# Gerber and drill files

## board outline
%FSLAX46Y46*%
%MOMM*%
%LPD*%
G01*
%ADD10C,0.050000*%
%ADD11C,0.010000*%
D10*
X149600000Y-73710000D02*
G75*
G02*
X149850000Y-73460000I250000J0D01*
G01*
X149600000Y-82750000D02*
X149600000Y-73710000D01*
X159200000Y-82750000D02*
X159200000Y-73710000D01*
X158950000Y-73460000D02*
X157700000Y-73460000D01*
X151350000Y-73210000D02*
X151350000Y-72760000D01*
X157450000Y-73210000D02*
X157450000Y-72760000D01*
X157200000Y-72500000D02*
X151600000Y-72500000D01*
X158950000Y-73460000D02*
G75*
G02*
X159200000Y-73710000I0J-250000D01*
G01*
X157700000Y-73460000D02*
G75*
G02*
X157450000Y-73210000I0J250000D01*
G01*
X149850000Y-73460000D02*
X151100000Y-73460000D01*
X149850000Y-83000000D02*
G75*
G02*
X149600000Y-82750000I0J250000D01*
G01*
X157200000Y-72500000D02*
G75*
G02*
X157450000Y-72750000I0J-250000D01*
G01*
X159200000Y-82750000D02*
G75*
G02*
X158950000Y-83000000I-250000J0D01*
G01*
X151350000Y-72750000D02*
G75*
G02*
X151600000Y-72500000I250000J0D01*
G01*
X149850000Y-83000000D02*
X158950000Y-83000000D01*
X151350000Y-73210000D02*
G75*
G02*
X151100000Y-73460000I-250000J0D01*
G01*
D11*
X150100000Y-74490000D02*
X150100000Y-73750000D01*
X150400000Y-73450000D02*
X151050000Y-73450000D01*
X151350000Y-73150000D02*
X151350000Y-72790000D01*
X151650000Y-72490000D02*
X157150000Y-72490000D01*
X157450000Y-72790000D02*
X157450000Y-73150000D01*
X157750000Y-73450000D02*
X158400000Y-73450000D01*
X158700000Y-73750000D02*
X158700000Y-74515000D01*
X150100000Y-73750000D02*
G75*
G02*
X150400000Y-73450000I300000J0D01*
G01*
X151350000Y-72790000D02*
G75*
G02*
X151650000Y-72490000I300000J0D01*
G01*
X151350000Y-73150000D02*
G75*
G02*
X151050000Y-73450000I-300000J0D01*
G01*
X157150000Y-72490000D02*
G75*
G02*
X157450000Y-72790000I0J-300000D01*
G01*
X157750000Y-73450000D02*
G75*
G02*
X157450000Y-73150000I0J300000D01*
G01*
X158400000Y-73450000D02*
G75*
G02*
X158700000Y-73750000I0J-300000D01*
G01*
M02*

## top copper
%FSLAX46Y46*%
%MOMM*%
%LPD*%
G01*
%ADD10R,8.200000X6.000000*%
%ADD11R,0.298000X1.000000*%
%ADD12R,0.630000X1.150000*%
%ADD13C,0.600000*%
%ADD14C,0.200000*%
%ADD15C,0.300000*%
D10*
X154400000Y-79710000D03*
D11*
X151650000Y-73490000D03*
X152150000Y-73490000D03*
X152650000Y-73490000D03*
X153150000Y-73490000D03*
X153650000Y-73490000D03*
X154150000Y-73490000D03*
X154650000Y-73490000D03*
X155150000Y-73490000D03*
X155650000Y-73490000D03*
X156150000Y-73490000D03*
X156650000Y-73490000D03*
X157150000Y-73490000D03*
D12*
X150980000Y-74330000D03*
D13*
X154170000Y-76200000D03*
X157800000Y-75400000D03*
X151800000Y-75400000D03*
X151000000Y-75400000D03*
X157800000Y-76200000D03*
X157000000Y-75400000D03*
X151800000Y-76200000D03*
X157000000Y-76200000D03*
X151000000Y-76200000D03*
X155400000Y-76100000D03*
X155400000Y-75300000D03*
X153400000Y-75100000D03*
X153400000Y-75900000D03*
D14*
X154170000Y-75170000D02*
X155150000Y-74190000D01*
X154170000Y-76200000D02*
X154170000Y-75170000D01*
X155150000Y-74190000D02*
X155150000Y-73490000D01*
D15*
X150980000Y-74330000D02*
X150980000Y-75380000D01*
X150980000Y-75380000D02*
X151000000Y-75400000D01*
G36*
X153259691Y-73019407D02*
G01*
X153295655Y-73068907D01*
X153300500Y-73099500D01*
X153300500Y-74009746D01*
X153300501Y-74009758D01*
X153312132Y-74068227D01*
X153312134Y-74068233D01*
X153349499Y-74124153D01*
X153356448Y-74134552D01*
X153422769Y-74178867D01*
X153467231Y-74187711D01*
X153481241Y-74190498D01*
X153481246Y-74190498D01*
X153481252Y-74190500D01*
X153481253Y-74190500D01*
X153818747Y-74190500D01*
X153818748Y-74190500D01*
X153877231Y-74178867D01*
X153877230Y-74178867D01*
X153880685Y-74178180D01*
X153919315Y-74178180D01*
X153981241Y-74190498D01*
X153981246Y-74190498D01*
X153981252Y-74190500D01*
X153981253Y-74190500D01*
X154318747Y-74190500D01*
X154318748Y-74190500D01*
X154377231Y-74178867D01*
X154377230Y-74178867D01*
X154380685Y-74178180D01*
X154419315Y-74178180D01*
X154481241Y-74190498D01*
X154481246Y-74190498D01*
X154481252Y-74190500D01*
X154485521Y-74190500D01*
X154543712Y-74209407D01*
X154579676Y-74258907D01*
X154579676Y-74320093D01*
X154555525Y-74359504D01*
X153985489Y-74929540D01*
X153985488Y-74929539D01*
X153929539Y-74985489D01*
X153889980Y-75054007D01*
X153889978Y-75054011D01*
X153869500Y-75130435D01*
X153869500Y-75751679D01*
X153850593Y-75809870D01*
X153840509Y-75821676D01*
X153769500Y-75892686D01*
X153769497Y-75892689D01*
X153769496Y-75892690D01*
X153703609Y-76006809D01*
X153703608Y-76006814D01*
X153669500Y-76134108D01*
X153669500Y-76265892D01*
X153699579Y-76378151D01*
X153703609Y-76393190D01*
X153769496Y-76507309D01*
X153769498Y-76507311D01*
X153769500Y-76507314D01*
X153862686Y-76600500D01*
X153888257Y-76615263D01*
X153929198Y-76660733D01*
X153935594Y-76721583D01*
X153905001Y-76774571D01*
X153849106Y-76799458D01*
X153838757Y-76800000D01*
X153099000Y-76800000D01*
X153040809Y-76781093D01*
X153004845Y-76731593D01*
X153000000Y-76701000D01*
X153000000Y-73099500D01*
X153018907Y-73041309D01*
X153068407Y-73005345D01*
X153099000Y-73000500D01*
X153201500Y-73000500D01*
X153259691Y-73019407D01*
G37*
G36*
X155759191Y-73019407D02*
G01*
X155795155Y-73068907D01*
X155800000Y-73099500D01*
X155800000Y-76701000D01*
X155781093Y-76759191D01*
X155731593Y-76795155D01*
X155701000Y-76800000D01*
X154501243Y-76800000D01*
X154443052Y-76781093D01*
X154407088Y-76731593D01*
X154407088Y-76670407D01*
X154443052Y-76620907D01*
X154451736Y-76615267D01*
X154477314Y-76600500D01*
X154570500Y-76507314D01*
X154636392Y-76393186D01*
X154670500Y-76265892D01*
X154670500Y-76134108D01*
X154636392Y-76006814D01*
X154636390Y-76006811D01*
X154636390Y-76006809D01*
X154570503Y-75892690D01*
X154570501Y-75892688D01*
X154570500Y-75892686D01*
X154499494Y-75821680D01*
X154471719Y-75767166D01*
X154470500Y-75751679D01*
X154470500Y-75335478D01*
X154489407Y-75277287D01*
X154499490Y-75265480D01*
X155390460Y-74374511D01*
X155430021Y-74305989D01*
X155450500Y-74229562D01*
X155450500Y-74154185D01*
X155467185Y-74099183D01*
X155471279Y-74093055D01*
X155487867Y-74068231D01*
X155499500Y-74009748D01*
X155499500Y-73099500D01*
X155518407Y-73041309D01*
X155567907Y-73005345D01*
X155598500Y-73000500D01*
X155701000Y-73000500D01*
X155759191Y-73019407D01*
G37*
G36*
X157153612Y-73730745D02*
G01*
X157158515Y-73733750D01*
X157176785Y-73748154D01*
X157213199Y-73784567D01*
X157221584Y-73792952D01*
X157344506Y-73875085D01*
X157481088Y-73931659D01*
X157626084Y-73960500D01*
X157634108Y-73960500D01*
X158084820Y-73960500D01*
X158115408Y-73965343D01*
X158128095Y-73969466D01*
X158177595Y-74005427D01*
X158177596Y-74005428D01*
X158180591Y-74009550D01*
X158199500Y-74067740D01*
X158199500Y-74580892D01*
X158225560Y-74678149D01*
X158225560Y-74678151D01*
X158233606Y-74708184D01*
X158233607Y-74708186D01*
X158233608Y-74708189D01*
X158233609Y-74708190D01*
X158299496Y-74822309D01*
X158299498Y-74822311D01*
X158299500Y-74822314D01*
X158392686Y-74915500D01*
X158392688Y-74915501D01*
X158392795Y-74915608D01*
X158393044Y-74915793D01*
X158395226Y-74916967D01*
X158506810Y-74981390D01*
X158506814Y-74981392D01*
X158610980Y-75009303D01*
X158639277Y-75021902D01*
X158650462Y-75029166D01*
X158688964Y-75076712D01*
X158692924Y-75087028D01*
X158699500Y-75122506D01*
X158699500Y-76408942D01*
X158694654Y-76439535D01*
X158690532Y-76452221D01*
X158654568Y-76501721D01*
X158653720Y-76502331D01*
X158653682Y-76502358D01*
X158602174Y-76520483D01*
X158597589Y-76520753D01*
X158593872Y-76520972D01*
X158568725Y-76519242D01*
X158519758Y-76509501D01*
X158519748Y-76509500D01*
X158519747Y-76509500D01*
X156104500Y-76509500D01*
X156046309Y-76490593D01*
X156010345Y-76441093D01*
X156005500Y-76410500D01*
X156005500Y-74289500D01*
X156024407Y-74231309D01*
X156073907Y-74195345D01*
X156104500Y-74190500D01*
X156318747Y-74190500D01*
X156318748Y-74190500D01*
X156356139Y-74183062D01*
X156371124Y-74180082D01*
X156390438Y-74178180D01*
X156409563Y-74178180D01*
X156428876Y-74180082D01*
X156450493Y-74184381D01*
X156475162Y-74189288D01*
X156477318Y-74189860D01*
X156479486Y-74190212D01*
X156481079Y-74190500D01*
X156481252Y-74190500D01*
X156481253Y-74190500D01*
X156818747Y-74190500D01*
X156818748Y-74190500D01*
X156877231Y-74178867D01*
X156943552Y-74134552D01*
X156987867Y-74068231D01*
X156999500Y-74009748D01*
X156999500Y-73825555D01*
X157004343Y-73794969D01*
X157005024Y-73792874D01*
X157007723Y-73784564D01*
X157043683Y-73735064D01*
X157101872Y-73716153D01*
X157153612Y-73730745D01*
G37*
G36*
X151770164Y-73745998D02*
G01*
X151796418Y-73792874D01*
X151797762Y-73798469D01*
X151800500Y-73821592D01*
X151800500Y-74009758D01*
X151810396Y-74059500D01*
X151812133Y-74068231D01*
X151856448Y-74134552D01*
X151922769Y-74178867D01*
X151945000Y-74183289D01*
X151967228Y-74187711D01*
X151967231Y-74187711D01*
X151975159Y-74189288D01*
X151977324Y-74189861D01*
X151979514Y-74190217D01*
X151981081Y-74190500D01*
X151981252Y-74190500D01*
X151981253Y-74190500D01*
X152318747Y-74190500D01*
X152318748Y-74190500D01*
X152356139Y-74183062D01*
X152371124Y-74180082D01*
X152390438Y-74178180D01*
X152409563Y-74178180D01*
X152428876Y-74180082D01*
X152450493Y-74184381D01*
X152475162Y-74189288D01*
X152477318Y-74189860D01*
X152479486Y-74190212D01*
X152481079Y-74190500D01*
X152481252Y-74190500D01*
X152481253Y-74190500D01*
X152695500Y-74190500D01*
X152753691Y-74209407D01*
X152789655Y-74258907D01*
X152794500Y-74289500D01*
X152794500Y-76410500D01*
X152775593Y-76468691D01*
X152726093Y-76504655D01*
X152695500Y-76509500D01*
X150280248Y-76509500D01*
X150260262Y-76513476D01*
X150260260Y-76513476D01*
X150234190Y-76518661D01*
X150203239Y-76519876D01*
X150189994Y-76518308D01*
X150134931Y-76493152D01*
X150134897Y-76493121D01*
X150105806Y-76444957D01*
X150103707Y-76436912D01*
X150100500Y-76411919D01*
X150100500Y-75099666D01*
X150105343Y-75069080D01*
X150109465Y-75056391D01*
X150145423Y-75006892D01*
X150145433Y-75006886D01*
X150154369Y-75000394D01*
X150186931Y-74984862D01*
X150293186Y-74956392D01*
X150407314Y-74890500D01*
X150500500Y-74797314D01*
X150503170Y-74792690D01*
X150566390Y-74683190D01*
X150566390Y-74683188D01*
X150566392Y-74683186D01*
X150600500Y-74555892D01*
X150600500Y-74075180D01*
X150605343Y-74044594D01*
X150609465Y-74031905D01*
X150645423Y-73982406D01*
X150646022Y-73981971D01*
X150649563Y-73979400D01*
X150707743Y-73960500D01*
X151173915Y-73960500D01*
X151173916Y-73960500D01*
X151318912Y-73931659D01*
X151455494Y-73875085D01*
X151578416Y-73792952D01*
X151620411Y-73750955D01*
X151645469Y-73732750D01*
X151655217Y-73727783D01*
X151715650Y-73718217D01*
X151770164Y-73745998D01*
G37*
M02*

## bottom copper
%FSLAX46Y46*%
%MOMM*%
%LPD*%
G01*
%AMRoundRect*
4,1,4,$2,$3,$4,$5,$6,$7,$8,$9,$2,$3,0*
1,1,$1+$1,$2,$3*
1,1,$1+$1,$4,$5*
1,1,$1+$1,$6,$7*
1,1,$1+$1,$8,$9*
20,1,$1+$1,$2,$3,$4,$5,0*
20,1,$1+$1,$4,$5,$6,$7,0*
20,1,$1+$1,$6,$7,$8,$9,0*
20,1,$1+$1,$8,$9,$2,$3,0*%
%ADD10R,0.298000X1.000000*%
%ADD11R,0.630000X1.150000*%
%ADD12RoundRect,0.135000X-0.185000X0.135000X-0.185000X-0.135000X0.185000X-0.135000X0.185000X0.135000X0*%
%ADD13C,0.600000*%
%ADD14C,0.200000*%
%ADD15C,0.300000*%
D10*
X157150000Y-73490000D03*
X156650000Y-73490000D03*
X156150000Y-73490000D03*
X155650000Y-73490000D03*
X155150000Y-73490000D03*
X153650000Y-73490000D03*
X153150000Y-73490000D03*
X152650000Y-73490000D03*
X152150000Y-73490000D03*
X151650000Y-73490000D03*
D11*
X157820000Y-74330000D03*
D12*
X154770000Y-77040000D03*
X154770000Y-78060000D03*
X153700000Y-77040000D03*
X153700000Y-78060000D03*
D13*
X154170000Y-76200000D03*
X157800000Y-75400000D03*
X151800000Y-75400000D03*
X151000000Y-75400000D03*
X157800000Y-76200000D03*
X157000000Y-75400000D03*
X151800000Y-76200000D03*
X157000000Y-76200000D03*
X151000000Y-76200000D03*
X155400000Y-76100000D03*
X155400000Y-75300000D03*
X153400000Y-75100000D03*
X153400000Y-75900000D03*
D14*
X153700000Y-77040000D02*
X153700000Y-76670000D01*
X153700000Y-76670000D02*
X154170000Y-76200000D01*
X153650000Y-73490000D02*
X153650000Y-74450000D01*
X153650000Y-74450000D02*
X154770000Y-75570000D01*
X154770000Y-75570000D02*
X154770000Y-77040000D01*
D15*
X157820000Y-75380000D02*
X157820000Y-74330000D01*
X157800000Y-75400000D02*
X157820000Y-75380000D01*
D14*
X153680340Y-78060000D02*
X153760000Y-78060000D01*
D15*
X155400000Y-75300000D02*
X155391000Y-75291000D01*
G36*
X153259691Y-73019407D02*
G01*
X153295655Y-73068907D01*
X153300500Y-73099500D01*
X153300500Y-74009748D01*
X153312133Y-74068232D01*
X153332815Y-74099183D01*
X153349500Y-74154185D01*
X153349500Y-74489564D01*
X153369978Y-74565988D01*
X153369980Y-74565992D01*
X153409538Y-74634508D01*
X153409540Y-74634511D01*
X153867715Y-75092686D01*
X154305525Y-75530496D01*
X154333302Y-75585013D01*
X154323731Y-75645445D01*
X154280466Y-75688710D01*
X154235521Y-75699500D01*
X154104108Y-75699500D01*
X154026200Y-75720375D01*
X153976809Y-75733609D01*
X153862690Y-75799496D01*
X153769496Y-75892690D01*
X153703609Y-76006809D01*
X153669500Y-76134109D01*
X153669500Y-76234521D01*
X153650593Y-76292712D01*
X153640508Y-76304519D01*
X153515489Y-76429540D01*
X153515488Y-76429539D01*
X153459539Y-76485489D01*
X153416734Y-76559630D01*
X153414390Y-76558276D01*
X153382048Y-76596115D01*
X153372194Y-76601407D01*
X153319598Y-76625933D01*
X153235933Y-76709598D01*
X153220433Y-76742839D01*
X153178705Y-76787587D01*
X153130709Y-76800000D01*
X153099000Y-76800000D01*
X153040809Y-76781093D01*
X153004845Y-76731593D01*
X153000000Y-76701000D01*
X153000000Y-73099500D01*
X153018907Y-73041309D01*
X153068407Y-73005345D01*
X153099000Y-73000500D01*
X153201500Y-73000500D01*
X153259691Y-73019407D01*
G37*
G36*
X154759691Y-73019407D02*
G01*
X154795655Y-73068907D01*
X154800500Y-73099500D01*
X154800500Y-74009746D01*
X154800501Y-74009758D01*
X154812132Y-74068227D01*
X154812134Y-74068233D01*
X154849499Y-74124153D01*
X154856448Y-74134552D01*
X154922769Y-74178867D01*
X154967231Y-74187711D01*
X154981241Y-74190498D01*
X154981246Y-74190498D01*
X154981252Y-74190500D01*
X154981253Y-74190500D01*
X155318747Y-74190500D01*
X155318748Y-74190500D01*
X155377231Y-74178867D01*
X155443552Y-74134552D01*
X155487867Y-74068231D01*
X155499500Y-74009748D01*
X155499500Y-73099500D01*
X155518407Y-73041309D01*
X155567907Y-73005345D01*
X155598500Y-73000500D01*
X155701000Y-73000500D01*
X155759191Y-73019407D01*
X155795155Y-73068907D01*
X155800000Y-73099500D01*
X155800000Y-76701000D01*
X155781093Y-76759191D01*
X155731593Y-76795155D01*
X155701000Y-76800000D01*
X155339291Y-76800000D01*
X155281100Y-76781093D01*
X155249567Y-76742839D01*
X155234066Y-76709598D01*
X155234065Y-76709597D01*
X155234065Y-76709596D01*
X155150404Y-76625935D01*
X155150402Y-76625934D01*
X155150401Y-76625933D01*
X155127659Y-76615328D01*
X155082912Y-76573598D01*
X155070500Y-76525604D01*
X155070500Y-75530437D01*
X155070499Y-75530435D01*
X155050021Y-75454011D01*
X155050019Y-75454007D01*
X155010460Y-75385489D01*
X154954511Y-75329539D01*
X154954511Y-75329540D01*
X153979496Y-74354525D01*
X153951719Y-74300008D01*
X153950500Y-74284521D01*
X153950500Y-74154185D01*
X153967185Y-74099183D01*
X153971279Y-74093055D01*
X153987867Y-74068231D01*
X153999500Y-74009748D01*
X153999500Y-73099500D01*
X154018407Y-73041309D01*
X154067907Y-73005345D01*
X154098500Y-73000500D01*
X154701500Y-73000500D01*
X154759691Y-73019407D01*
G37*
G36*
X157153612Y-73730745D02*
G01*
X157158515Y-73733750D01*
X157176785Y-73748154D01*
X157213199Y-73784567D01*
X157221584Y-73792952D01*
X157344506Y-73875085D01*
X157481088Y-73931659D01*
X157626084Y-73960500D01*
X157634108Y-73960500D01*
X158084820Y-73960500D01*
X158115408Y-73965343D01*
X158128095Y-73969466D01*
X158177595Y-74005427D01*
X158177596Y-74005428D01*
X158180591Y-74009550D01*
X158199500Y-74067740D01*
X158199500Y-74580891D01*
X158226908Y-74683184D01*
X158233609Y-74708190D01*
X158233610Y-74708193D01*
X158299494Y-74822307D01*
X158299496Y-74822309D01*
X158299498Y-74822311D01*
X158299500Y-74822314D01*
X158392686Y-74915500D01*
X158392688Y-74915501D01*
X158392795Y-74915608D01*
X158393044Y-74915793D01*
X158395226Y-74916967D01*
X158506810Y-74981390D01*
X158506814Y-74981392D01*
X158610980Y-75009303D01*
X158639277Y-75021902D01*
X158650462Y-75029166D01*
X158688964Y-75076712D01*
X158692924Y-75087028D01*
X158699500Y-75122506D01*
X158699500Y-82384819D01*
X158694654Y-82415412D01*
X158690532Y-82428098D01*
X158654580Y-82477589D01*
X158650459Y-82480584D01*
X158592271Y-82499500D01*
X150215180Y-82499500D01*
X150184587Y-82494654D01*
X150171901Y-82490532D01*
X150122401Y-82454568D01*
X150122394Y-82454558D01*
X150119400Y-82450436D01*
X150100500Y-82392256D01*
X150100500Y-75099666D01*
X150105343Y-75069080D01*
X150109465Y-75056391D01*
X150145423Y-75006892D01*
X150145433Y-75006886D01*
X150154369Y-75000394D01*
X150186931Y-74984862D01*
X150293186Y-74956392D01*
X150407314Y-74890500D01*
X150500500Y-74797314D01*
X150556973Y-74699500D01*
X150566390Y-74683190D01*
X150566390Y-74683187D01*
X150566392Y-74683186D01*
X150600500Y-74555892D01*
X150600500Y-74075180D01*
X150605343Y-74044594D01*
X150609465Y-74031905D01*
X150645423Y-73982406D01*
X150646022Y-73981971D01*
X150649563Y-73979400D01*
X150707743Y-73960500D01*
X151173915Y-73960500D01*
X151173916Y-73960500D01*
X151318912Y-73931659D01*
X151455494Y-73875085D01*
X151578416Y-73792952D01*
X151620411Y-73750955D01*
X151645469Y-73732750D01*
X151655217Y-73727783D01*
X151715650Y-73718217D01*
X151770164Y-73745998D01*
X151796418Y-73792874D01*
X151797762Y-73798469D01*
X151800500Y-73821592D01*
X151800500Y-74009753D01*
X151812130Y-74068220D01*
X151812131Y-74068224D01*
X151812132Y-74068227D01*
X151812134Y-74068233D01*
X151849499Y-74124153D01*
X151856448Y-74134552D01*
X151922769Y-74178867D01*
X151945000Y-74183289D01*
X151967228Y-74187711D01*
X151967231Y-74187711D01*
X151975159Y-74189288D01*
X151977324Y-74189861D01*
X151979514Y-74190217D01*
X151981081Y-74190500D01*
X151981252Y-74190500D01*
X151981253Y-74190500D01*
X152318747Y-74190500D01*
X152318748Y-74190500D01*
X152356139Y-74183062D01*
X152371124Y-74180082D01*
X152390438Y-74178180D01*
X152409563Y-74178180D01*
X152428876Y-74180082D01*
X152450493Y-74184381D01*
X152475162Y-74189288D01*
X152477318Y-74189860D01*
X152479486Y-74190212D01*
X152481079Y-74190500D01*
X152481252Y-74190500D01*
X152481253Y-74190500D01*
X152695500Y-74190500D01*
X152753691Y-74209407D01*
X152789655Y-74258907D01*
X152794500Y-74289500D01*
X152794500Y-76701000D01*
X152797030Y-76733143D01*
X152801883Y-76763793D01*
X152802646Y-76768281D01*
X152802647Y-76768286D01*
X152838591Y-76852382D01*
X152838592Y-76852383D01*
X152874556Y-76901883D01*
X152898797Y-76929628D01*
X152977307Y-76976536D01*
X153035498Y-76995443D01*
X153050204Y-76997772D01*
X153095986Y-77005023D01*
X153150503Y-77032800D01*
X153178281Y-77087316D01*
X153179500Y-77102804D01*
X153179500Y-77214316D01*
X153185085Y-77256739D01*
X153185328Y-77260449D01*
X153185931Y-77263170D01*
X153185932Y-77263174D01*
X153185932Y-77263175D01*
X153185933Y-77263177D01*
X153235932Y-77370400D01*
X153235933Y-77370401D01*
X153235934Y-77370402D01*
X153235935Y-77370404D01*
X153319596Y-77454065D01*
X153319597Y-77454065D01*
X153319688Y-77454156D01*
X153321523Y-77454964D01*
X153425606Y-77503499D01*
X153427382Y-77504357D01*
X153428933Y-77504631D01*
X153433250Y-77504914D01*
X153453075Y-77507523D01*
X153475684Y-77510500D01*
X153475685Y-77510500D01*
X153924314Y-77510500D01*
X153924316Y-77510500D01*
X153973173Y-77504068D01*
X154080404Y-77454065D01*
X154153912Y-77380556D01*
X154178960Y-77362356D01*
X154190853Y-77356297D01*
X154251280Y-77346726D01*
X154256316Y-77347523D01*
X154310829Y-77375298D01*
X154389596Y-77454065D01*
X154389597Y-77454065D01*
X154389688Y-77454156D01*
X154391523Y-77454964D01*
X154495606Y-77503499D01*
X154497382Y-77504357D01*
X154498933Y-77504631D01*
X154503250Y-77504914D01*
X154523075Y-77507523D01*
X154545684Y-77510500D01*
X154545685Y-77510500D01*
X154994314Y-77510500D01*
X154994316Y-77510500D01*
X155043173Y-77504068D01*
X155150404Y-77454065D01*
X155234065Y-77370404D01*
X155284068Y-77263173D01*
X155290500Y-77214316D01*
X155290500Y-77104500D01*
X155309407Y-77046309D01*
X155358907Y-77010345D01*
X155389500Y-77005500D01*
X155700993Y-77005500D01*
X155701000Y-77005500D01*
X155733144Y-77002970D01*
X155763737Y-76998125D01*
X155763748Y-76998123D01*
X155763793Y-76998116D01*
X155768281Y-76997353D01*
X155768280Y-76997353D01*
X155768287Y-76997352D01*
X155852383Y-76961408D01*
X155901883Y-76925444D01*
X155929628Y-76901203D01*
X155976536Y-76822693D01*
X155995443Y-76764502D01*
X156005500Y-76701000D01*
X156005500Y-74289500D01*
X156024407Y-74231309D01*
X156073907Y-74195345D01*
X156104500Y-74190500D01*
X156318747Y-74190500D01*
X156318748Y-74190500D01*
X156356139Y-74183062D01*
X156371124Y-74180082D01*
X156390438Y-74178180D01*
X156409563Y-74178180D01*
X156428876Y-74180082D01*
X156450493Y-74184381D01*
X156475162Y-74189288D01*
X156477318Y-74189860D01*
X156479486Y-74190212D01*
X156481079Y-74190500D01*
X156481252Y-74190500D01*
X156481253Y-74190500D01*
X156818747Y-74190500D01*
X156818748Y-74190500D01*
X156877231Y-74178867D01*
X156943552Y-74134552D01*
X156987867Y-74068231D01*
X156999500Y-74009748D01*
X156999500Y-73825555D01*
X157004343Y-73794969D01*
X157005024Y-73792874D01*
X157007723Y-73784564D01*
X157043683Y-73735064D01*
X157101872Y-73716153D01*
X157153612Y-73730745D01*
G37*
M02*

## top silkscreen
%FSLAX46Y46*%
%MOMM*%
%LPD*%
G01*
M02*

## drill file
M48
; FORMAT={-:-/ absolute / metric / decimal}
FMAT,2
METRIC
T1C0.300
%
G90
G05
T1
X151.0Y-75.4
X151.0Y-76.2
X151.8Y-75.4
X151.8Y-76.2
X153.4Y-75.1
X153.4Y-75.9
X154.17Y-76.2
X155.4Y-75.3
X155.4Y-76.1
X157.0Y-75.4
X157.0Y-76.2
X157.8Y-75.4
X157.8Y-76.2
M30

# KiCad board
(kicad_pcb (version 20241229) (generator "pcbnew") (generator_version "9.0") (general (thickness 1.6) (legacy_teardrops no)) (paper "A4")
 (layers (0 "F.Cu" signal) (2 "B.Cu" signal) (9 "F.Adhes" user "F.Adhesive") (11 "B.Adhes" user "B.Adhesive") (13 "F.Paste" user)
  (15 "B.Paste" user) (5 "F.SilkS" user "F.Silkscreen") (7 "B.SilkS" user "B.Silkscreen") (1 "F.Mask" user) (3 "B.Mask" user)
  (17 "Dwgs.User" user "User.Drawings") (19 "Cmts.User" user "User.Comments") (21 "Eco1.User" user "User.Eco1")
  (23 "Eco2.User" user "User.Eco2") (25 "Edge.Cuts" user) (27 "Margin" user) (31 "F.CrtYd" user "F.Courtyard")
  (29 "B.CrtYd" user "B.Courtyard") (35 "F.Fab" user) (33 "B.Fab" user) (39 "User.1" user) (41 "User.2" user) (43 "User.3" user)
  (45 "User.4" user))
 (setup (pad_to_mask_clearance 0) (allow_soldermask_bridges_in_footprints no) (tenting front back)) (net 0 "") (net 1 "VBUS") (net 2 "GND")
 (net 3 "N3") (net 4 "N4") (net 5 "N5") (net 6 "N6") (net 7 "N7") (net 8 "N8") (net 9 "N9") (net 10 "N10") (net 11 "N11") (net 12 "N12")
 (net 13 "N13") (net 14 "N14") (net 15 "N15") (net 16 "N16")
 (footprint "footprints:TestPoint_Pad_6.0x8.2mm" (layer "F.Cu") (at 154.3 79.81)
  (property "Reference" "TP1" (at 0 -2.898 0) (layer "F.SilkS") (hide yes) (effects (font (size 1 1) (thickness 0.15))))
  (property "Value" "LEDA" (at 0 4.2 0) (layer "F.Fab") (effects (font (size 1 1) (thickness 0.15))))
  (pad "1" smd rect (at 0.1 -0.1) (size 8.2 6) (layers "F.Cu" "F.Mask") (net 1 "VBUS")))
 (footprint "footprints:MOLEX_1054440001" (layer "F.Cu") (at 154.4 72.49 180)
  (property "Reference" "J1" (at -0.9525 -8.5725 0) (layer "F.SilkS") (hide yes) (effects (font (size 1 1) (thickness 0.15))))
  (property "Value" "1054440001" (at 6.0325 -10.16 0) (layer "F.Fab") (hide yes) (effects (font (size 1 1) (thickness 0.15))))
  (fp_line (start 4.3 -2) (end 4.3 -1.26) (stroke (width 0.01) (type solid)) (layer "Edge.Cuts"))
  (fp_line (start 4 -0.96) (end 3.35 -0.96) (stroke (width 0.01) (type solid)) (layer "Edge.Cuts"))
  (fp_line (start 3.05 -0.66) (end 3.05 -0.3) (stroke (width 0.01) (type solid)) (layer "Edge.Cuts"))
  (fp_line (start 2.75 0) (end -2.75 0) (stroke (width 0.01) (type solid)) (layer "Edge.Cuts"))
  (fp_line (start -3.05 -0.3) (end -3.05 -0.66) (stroke (width 0.01) (type solid)) (layer "Edge.Cuts"))
  (fp_line (start -3.35 -0.96) (end -4 -0.96) (stroke (width 0.01) (type solid)) (layer "Edge.Cuts"))
  (fp_line (start -4.3 -1.26) (end -4.3 -2.025) (stroke (width 0.01) (type solid)) (layer "Edge.Cuts"))
  (fp_arc (start 4.3 -1.26) (mid 4.212132 -1.047868) (end 4 -0.96) (stroke (width 0.01) (type solid)) (layer "Edge.Cuts"))
  (fp_arc (start 3.05 -0.3) (mid 2.962132 -0.087868) (end 2.75 0) (stroke (width 0.01) (type solid)) (layer "Edge.Cuts"))
  (fp_arc (start 3.05 -0.66) (mid 3.137868 -0.872132) (end 3.35 -0.96) (stroke (width 0.01) (type solid)) (layer "Edge.Cuts"))
  (fp_arc (start -2.75 0) (mid -2.962132 -0.087868) (end -3.05 -0.3) (stroke (width 0.01) (type solid)) (layer "Edge.Cuts"))
  (fp_arc (start -3.35 -0.96) (mid -3.137868 -0.872132) (end -3.05 -0.66) (stroke (width 0.01) (type solid)) (layer "Edge.Cuts"))
  (fp_arc (start -4 -0.96) (mid -4.212132 -1.047868) (end -4.3 -1.26) (stroke (width 0.01) (type solid)) (layer "Edge.Cuts"))
  (pad "A1" smd rect (at 2.75 -1 180) (size 0.298 1) (layers "F.Cu" "F.Paste") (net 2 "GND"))
  (pad "A2" smd rect (at 2.25 -1 180) (size 0.298 1) (layers "F.Cu" "F.Paste") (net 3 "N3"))
  (pad "A3" smd rect (at 1.75 -1 180) (size 0.298 1) (layers "F.Cu" "F.Paste") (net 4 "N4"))
  (pad "A4" smd rect (at 1.25 -1 180) (size 0.298 1) (layers "F.Cu" "F.Paste") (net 1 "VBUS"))
  (pad "A5" smd rect (at 0.75 -1 180) (size 0.298 1) (layers "F.Cu" "F.Paste") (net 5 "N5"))
  (pad "A6" smd rect (at 0.25 -1 180) (size 0.298 1) (layers "F.Cu" "F.Paste") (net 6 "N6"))
  (pad "A7" smd rect (at -0.25 -1 180) (size 0.298 1) (layers "F.Cu" "F.Paste") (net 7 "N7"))
  (pad "A8" smd rect (at -0.75 -1 180) (size 0.298 1) (layers "F.Cu" "F.Paste") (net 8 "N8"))
  (pad "A9" smd rect (at -1.25 -1 180) (size 0.298 1) (layers "F.Cu" "F.Paste") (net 1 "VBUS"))
  (pad "A10" smd rect (at -1.75 -1 180) (size 0.298 1) (layers "F.Cu" "F.Paste") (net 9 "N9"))
  (pad "A11" smd rect (at -2.25 -1 180) (size 0.298 1) (layers "F.Cu" "F.Paste") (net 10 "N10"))
  (pad "A12" smd rect (at -2.75 -1 180) (size 0.298 1) (layers "F.Cu" "F.Paste") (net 2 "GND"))
  (pad "B1" smd rect (at -2.75 -1 180) (size 0.298 1) (layers "B.Cu" "B.Paste") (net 2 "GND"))
  (pad "B2" smd rect (at -2.25 -1 180) (size 0.298 1) (layers "B.Cu" "B.Paste") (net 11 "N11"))
  (pad "B3" smd rect (at -1.75 -1 180) (size 0.298 1) (layers "B.Cu" "B.Paste") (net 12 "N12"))
  (pad "B4" smd rect (at -1.25 -1 180) (size 0.298 1) (layers "B.Cu" "B.Paste") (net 1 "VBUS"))
  (pad "B5" smd rect (at -0.75 -1 180) (size 0.298 1) (layers "B.Cu" "B.Paste") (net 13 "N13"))
  (pad "B8" smd rect (at 0.75 -1 180) (size 0.298 1) (layers "B.Cu" "B.Paste") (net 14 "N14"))
  (pad "B9" smd rect (at 1.25 -1 180) (size 0.298 1) (layers "B.Cu" "B.Paste") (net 1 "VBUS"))
  (pad "B10" smd rect (at 1.75 -1 180) (size 0.298 1) (layers "B.Cu" "B.Paste") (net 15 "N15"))
  (pad "B11" smd rect (at 2.25 -1 180) (size 0.298 1) (layers "B.Cu" "B.Paste") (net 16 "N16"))
  (pad "B12" smd rect (at 2.75 -1 180) (size 0.298 1) (layers "B.Cu" "B.Paste") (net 2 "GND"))
  (pad "SH1" smd rect (at 3.42 -1.84 180) (size 0.63 1.15) (layers "F.Cu" "F.Paste") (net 2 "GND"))
  (pad "SH2" smd rect (at -3.42 -1.84 180) (size 0.63 1.15) (layers "B.Cu" "B.Paste") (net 2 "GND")))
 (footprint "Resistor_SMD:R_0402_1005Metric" (layer "B.Cu") (at 154.77 77.55 -90)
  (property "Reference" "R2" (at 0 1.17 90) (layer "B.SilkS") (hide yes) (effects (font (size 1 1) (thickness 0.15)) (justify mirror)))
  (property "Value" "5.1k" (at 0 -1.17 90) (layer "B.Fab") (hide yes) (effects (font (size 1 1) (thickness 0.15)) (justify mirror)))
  (pad "1" smd roundrect (at -0.51 0 270) (size 0.54 0.64) (layers "B.Cu" "B.Mask" "B.Paste") (roundrect_rratio 0.25) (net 14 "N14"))
  (pad "2" smd roundrect (at 0.51 0 270) (size 0.54 0.64) (layers "B.Cu" "B.Mask" "B.Paste") (roundrect_rratio 0.25) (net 2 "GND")))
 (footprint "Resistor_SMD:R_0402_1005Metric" (layer "B.Cu") (at 153.7 77.55 -90)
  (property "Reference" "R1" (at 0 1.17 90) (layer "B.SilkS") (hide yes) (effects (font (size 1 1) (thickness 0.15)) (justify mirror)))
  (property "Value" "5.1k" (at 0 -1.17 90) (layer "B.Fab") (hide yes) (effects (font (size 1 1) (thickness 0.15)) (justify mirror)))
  (pad "1" smd roundrect (at -0.51 0 270) (size 0.54 0.64) (layers "B.Cu" "B.Mask" "B.Paste") (roundrect_rratio 0.25) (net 8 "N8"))
  (pad "2" smd roundrect (at 0.51 0 270) (size 0.54 0.64) (layers "B.Cu" "B.Mask" "B.Paste") (roundrect_rratio 0.25) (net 2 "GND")))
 (gr_arc (start 149.6 73.71) (mid 149.673223 73.533223) (end 149.85 73.46) (stroke (width 0.05) (type default)) (layer "Edge.Cuts"))
 (gr_line (start 149.6 82.75) (end 149.6 73.71) (stroke (width 0.05) (type solid)) (layer "Edge.Cuts"))
 (gr_line (start 159.2 82.75) (end 159.2 73.71) (stroke (width 0.05) (type solid)) (layer "Edge.Cuts"))
 (gr_line (start 158.95 73.46) (end 157.7 73.46) (stroke (width 0.05) (type solid)) (layer "Edge.Cuts"))
 (gr_line (start 151.35 73.21) (end 151.35 72.76) (stroke (width 0.05) (type solid)) (layer "Edge.Cuts"))
 (gr_line (start 157.45 73.21) (end 157.45 72.76) (stroke (width 0.05) (type solid)) (layer "Edge.Cuts"))
 (gr_line (start 157.2 72.5) (end 151.6 72.5) (stroke (width 0.05) (type default)) (layer "Edge.Cuts"))
 (gr_arc (start 158.95 73.46) (mid 159.126777 73.533223) (end 159.2 73.71) (stroke (width 0.05) (type default)) (layer "Edge.Cuts"))
 (gr_arc (start 157.7 73.46) (mid 157.523223 73.386777) (end 157.45 73.21) (stroke (width 0.05) (type default)) (layer "Edge.Cuts"))
 (gr_line (start 149.85 73.46) (end 151.1 73.46) (stroke (width 0.05) (type solid)) (layer "Edge.Cuts"))
 (gr_arc (start 149.85 83) (mid 149.673223 82.926777) (end 149.6 82.75) (stroke (width 0.05) (type default)) (layer "Edge.Cuts"))
 (gr_arc (start 157.2 72.5) (mid 157.376777 72.573223) (end 157.45 72.75) (stroke (width 0.05) (type default)) (layer "Edge.Cuts"))
 (gr_arc (start 159.2 82.75) (mid 159.126777 82.926777) (end 158.95 83) (stroke (width 0.05) (type default)) (layer "Edge.Cuts"))
 (gr_arc (start 151.35 72.75) (mid 151.423223 72.573223) (end 151.6 72.5) (stroke (width 0.05) (type default)) (layer "Edge.Cuts"))
 (gr_line (start 149.85 83) (end 158.95 83) (stroke (width 0.05) (type default)) (layer "Edge.Cuts"))
 (gr_arc (start 151.35 73.21) (mid 151.276777 73.386777) (end 151.1 73.46) (stroke (width 0.05) (type default)) (layer "Edge.Cuts"))
 (segment (start 154.17 75.17) (end 155.15 74.19) (width 0.2) (layer "F.Cu") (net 8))
 (segment (start 154.17 76.2) (end 154.17 75.17) (width 0.2) (layer "F.Cu") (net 8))
 (segment (start 155.15 74.19) (end 155.15 73.49) (width 0.2) (layer "F.Cu") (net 8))
 (via (at 154.17 76.2) (size 0.6) (drill 0.3) (layers "F.Cu" "B.Cu") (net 8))
 (segment (start 153.7 77.04) (end 153.7 76.67) (width 0.2) (layer "B.Cu") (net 8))
 (segment (start 153.7 76.67) (end 154.17 76.2) (width 0.2) (layer "B.Cu") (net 8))
 (segment (start 153.65 73.49) (end 153.65 74.45) (width 0.2) (layer "B.Cu") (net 14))
 (segment (start 153.65 74.45) (end 154.77 75.57) (width 0.2) (layer "B.Cu") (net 14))
 (segment (start 154.77 75.57) (end 154.77 77.04) (width 0.2) (layer "B.Cu") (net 14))
 (segment (start 150.98 74.33) (end 150.98 75.38) (width 0.3) (layer "F.Cu") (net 2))
 (segment (start 150.98 75.38) (end 151 75.4) (width 0.3) (layer "F.Cu") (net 2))
 (via (at 157.8 75.4) (size 0.6) (drill 0.3) (layers "F.Cu" "B.Cu") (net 2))
 (via (at 151.8 75.4) (size 0.6) (drill 0.3) (layers "F.Cu" "B.Cu") (free yes) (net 2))
 (via (at 151 75.4) (size 0.6) (drill 0.3) (layers "F.Cu" "B.Cu") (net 2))
 (via (at 157.8 76.2) (size 0.6) (drill 0.3) (layers "F.Cu" "B.Cu") (free yes) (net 2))
 (via (at 157 75.4) (size 0.6) (drill 0.3) (layers "F.Cu" "B.Cu") (free yes) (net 2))
 (via (at 151.8 76.2) (size 0.6) (drill 0.3) (layers "F.Cu" "B.Cu") (free yes) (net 2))
 (via (at 157 76.2) (size 0.6) (drill 0.3) (layers "F.Cu" "B.Cu") (free yes) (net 2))
 (via (at 151 76.2) (size 0.6) (drill 0.3) (layers "F.Cu" "B.Cu") (free yes) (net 2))
 (segment (start 157.82 75.38) (end 157.82 74.33) (width 0.3) (layer "B.Cu") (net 2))
 (segment (start 157.8 75.4) (end 157.82 75.38) (width 0.3) (layer "B.Cu") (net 2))
 (segment (start 153.68034 78.06) (end 153.76 78.06) (width 0.2) (layer "B.Cu") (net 2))
 (via (at 155.4 76.1) (size 0.6) (drill 0.3) (layers "F.Cu" "B.Cu") (free yes) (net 1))
 (via (at 155.4 75.3) (size 0.6) (drill 0.3) (layers "F.Cu" "B.Cu") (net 1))
 (via (at 153.4 75.1) (size 0.6) (drill 0.3) (layers "F.Cu" "B.Cu") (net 1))
 (via (at 153.4 75.9) (size 0.6) (drill 0.3) (layers "F.Cu" "B.Cu") (free yes) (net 1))
 (segment (start 155.4 75.3) (end 155.391 75.291) (width 0.3) (layer "B.Cu") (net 1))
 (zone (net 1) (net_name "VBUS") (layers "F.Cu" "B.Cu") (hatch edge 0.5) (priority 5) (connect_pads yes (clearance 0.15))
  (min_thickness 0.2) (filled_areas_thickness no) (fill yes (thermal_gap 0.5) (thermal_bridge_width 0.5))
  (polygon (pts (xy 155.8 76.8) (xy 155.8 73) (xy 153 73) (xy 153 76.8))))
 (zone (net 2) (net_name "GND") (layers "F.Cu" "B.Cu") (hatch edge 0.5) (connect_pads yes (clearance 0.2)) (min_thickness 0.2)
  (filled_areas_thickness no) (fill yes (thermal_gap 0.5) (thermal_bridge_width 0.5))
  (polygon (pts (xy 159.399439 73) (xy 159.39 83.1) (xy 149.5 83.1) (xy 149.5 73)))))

